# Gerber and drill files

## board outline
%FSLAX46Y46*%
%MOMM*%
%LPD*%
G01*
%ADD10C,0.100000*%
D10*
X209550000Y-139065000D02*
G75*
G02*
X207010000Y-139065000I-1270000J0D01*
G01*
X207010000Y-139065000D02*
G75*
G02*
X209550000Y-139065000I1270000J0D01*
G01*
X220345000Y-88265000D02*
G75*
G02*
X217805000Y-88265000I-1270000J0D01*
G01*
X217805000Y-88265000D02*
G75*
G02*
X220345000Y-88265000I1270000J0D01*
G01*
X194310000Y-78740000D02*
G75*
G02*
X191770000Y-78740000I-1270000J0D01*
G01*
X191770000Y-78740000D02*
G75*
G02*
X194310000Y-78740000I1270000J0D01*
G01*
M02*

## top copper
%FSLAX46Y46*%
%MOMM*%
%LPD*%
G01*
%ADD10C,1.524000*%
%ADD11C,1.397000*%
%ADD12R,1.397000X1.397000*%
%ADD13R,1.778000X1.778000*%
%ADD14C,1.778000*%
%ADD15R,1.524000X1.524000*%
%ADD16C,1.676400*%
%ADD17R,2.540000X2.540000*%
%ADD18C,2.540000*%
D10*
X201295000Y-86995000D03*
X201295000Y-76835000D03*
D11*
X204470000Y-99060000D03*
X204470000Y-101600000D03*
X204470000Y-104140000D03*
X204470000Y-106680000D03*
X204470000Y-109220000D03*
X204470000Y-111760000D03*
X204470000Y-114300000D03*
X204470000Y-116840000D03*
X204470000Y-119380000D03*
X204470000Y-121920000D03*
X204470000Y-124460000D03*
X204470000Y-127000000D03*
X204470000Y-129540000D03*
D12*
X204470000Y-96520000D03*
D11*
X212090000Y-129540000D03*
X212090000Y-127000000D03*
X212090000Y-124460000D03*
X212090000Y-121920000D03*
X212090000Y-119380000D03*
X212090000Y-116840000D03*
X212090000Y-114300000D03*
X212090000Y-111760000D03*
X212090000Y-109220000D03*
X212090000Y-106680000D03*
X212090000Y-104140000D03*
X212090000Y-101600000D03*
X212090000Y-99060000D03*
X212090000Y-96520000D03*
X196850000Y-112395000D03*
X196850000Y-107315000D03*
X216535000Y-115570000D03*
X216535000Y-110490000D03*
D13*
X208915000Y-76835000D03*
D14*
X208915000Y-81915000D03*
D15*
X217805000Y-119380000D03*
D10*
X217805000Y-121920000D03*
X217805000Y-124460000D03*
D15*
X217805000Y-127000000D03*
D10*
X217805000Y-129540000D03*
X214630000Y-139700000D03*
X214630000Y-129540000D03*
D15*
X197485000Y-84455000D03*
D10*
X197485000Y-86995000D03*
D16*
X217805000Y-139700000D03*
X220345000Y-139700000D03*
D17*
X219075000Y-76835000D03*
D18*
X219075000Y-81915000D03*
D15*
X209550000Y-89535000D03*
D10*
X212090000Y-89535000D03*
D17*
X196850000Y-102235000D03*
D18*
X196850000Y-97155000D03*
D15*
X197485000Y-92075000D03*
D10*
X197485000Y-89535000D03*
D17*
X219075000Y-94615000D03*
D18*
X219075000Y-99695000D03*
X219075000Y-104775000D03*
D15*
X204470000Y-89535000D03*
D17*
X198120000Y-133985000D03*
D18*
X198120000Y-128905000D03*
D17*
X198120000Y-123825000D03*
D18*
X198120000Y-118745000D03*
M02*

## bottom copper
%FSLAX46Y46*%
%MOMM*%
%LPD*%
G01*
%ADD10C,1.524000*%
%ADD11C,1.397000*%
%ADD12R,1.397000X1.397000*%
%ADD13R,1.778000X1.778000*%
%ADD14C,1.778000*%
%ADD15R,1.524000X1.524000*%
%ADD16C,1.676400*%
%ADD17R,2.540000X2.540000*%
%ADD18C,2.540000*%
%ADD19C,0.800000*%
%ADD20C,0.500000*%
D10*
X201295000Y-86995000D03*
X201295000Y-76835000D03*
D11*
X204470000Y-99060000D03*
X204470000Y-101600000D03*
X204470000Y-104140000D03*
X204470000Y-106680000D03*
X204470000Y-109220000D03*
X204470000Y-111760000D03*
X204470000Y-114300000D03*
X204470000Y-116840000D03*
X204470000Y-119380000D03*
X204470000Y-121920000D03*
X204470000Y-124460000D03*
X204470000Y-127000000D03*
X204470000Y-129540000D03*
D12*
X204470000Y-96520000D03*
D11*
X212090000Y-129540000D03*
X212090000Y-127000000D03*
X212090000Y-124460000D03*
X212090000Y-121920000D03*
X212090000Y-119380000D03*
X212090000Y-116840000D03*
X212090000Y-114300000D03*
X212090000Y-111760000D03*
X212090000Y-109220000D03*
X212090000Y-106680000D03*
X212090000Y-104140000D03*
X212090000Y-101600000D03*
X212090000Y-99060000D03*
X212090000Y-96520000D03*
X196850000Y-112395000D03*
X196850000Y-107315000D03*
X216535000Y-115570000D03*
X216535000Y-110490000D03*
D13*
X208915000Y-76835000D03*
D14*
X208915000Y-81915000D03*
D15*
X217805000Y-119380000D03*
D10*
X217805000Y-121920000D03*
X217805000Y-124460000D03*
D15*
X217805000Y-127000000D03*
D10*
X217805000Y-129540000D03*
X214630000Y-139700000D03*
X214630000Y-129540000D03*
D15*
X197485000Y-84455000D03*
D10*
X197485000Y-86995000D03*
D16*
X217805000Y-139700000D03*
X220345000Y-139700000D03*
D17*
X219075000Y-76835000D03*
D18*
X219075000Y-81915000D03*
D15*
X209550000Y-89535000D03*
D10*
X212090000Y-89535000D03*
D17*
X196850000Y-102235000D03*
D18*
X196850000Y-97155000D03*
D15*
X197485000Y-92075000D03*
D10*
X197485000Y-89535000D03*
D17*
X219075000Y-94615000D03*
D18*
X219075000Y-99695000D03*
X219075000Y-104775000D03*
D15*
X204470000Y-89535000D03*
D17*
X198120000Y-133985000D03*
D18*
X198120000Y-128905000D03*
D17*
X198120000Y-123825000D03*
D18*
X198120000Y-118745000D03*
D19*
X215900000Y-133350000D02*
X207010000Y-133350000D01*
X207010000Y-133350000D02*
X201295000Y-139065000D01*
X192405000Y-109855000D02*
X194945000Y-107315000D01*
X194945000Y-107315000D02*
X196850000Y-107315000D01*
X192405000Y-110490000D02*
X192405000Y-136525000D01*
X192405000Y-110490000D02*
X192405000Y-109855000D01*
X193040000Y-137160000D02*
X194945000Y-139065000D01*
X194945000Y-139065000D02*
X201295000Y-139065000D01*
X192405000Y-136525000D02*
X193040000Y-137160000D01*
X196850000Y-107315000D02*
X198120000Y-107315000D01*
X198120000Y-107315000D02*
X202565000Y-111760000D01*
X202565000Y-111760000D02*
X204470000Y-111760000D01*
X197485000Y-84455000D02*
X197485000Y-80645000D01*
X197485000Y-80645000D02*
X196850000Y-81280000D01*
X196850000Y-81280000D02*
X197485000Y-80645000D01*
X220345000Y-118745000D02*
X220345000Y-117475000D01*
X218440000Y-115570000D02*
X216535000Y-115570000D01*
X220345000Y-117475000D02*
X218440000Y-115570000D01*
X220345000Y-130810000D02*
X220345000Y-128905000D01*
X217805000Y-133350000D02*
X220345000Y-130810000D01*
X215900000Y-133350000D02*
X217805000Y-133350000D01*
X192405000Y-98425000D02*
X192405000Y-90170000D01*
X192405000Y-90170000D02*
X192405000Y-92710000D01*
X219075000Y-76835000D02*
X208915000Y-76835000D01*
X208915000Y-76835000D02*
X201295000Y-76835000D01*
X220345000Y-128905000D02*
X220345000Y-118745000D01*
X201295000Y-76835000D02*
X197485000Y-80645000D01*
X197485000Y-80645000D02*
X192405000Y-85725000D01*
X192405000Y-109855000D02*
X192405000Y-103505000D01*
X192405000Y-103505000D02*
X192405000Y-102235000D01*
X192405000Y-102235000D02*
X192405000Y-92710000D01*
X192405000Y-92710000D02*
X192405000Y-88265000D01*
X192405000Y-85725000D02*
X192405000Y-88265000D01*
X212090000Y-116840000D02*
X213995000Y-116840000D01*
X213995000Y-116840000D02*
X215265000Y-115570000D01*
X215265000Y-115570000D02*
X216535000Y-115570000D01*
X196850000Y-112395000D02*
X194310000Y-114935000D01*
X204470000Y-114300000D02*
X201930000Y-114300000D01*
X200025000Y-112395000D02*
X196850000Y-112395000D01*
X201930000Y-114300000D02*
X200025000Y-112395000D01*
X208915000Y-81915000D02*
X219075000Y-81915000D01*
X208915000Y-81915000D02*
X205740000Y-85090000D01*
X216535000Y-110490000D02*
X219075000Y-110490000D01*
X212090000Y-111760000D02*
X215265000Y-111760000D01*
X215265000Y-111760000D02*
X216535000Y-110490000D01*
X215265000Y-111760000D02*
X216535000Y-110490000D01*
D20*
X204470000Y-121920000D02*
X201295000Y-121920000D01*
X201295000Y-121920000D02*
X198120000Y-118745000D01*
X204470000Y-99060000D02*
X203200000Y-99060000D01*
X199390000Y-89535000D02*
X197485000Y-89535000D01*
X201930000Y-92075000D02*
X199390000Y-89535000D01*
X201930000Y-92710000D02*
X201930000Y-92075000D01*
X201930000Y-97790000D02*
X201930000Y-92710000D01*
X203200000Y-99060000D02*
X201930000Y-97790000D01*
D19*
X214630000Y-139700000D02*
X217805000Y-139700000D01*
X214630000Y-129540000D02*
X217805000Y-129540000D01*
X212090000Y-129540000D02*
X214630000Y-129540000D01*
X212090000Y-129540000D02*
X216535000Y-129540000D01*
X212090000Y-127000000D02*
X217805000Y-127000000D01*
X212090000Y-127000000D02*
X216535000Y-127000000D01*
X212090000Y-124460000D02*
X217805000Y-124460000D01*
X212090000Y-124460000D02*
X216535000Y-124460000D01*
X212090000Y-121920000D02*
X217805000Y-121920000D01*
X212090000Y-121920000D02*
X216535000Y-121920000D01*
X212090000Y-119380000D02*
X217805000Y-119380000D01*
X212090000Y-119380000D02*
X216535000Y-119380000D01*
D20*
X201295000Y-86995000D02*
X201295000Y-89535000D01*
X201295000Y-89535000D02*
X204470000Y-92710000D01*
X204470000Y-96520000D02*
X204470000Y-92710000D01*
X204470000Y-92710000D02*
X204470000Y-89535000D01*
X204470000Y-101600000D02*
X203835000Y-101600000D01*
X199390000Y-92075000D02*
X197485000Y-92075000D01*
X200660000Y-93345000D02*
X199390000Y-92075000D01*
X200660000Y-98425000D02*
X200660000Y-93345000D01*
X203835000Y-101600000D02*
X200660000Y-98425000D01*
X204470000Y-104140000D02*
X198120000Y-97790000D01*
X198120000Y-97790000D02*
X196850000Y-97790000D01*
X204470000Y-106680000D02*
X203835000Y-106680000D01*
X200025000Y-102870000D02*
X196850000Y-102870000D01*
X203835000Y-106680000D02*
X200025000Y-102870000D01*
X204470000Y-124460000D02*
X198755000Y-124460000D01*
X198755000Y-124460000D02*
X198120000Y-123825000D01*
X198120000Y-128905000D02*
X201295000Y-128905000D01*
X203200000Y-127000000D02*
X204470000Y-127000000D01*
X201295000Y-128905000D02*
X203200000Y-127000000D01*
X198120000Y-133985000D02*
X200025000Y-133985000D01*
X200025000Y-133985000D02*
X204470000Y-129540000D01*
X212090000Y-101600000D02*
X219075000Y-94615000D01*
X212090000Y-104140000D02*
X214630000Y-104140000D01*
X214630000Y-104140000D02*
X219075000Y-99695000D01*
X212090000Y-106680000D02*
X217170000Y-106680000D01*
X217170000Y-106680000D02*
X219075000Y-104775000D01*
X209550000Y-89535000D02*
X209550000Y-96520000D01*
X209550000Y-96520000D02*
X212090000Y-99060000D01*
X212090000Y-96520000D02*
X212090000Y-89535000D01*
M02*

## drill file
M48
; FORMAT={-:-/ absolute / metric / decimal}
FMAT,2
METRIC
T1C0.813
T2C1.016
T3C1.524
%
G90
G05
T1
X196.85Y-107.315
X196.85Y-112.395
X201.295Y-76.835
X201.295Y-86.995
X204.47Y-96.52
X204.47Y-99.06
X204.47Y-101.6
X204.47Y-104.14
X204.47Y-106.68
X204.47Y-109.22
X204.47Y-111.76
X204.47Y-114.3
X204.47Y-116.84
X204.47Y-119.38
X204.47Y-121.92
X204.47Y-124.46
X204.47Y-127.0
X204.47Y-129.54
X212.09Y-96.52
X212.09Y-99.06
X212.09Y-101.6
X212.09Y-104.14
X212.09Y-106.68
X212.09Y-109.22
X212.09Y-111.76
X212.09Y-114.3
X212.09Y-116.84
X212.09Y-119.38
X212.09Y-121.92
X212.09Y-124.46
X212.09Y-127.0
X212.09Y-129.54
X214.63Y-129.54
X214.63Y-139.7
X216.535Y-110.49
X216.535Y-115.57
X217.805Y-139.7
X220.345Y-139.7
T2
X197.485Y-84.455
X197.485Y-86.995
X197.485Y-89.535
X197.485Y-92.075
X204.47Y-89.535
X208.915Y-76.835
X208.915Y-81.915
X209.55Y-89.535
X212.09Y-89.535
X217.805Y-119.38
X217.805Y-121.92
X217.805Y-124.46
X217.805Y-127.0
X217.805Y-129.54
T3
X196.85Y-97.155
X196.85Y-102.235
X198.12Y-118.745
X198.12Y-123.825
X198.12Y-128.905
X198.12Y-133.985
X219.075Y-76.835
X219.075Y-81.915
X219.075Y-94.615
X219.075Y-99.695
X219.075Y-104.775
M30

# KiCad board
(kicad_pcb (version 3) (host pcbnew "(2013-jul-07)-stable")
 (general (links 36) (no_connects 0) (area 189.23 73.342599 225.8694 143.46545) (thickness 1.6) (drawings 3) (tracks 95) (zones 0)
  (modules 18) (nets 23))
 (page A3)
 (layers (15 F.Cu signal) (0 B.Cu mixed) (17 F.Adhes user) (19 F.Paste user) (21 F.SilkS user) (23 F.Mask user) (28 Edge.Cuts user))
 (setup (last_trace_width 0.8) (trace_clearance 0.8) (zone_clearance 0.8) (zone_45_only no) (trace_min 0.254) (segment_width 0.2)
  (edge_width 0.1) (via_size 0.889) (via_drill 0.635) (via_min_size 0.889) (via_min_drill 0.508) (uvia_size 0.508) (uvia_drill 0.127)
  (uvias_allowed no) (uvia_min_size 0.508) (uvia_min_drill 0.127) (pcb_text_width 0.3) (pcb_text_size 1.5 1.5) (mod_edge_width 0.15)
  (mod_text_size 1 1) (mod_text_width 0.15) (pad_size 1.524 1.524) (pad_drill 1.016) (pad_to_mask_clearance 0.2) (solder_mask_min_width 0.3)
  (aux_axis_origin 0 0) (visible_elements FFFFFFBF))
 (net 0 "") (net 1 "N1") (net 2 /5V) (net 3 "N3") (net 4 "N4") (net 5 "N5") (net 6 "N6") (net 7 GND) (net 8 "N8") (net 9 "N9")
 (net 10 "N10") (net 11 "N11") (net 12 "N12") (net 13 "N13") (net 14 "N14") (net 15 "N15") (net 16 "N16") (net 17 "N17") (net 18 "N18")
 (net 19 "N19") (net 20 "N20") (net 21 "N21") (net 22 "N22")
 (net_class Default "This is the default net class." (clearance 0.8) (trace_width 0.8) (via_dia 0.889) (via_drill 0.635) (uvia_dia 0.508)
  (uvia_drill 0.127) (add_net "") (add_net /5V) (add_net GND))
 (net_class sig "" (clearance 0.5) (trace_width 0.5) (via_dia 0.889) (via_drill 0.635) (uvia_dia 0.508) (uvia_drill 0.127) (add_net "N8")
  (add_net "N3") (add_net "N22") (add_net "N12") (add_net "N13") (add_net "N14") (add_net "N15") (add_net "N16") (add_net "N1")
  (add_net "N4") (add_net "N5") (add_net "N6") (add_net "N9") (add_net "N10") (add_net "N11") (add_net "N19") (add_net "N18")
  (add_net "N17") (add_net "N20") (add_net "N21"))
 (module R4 (layer F.Cu) (at 201.295 81.915 90) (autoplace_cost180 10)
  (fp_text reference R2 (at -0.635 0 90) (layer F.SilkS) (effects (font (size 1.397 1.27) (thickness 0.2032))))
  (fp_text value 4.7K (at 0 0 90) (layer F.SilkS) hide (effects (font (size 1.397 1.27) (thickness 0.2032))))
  (pad 1 thru_hole circle (at -5.08 0 90) (size 1.524 1.524) (drill 0.8128) (layers *.Cu *.Mask F.SilkS) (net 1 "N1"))
  (pad 2 thru_hole circle (at 5.08 0 90) (size 1.524 1.524) (drill 0.8128) (layers *.Cu *.Mask F.SilkS) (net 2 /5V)))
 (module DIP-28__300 (layer F.Cu) (at 208.28 113.03 270)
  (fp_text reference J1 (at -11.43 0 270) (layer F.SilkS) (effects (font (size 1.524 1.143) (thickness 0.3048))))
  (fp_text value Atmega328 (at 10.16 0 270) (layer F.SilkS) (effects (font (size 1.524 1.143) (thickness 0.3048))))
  (pad 2 thru_hole circle (at -13.97 3.81 270) (size 1.397 1.397) (drill 0.8128) (layers *.Cu *.Mask F.SilkS) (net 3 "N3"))
  (pad 3 thru_hole circle (at -11.43 3.81 270) (size 1.397 1.397) (drill 0.8128) (layers *.Cu *.Mask F.SilkS) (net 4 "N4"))
  (pad 4 thru_hole circle (at -8.89 3.81 270) (size 1.397 1.397) (drill 0.8128) (layers *.Cu *.Mask F.SilkS) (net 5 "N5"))
  (pad 5 thru_hole circle (at -6.35 3.81 270) (size 1.397 1.397) (drill 0.8128) (layers *.Cu *.Mask F.SilkS) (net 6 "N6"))
  (pad 6 thru_hole circle (at -3.81 3.81 270) (size 1.397 1.397) (drill 0.8128) (layers *.Cu *.Mask F.SilkS))
  (pad 7 thru_hole circle (at -1.27 3.81 270) (size 1.397 1.397) (drill 0.8128) (layers *.Cu *.Mask F.SilkS) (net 2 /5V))
  (pad 8 thru_hole circle (at 1.27 3.81 270) (size 1.397 1.397) (drill 0.8128) (layers *.Cu *.Mask F.SilkS) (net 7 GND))
  (pad 9 thru_hole circle (at 3.81 3.81 270) (size 1.397 1.397) (drill 0.8128) (layers *.Cu *.Mask F.SilkS))
  (pad 10 thru_hole circle (at 6.35 3.81 270) (size 1.397 1.397) (drill 0.8128) (layers *.Cu *.Mask F.SilkS))
  (pad 11 thru_hole circle (at 8.89 3.81 270) (size 1.397 1.397) (drill 0.8128) (layers *.Cu *.Mask F.SilkS) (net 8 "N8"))
  (pad 12 thru_hole circle (at 11.43 3.81 270) (size 1.397 1.397) (drill 0.8128) (layers *.Cu *.Mask F.SilkS) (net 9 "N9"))
  (pad 13 thru_hole circle (at 13.97 3.81 270) (size 1.397 1.397) (drill 0.8128) (layers *.Cu *.Mask F.SilkS) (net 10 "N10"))
  (pad 14 thru_hole circle (at 16.51 3.81 270) (size 1.397 1.397) (drill 0.8128) (layers *.Cu *.Mask F.SilkS) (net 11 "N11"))
  (pad 1 thru_hole rect (at -16.51 3.81 270) (size 1.397 1.397) (drill 0.8128) (layers *.Cu *.Mask F.SilkS) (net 1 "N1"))
  (pad 15 thru_hole circle (at 16.51 -3.81 270) (size 1.397 1.397) (drill 0.8128) (layers *.Cu *.Mask F.SilkS) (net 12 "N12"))
  (pad 16 thru_hole circle (at 13.97 -3.81 270) (size 1.397 1.397) (drill 0.8128) (layers *.Cu *.Mask F.SilkS) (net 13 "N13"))
  (pad 17 thru_hole circle (at 11.43 -3.81 270) (size 1.397 1.397) (drill 0.8128) (layers *.Cu *.Mask F.SilkS) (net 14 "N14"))
  (pad 18 thru_hole circle (at 8.89 -3.81 270) (size 1.397 1.397) (drill 0.8128) (layers *.Cu *.Mask F.SilkS) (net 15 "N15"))
  (pad 19 thru_hole circle (at 6.35 -3.81 270) (size 1.397 1.397) (drill 0.8128) (layers *.Cu *.Mask F.SilkS) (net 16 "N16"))
  (pad 20 thru_hole circle (at 3.81 -3.81 270) (size 1.397 1.397) (drill 0.8128) (layers *.Cu *.Mask F.SilkS) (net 2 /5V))
  (pad 21 thru_hole circle (at 1.27 -3.81 270) (size 1.397 1.397) (drill 0.8128) (layers *.Cu *.Mask F.SilkS))
  (pad 22 thru_hole circle (at -1.27 -3.81 270) (size 1.397 1.397) (drill 0.8128) (layers *.Cu *.Mask F.SilkS) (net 7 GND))
  (pad 23 thru_hole circle (at -3.81 -3.81 270) (size 1.397 1.397) (drill 0.8128) (layers *.Cu *.Mask F.SilkS))
  (pad 24 thru_hole circle (at -6.35 -3.81 270) (size 1.397 1.397) (drill 0.8128) (layers *.Cu *.Mask F.SilkS) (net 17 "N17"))
  (pad 25 thru_hole circle (at -8.89 -3.81 270) (size 1.397 1.397) (drill 0.8128) (layers *.Cu *.Mask F.SilkS) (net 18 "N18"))
  (pad 26 thru_hole circle (at -11.43 -3.81 270) (size 1.397 1.397) (drill 0.8128) (layers *.Cu *.Mask F.SilkS) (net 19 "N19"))
  (pad 27 thru_hole circle (at -13.97 -3.81 270) (size 1.397 1.397) (drill 0.8128) (layers *.Cu *.Mask F.SilkS) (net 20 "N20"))
  (pad 28 thru_hole circle (at -16.51 -3.81 270) (size 1.397 1.397) (drill 0.8128) (layers *.Cu *.Mask F.SilkS) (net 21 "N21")))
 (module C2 (layer F.Cu) (at 196.85 109.855 90)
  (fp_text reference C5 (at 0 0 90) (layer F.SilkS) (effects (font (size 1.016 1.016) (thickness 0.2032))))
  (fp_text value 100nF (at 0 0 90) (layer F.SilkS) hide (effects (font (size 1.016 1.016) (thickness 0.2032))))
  (pad 1 thru_hole circle (at -2.54 0 90) (size 1.397 1.397) (drill 0.8128) (layers *.Cu *.Mask F.SilkS) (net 7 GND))
  (pad 2 thru_hole circle (at 2.54 0 90) (size 1.397 1.397) (drill 0.8128) (layers *.Cu *.Mask F.SilkS) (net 2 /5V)))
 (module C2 (layer F.Cu) (at 216.535 113.03 90)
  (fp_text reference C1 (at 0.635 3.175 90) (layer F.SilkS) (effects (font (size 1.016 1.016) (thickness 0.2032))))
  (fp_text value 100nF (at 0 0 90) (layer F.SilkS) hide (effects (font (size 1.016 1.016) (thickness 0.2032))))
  (pad 1 thru_hole circle (at -2.54 0 90) (size 1.397 1.397) (drill 0.8128) (layers *.Cu *.Mask F.SilkS) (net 2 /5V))
  (pad 2 thru_hole circle (at 2.54 0 90) (size 1.397 1.397) (drill 0.8128) (layers *.Cu *.Mask F.SilkS) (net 7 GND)))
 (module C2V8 (layer F.Cu) (at 208.915 79.375 270)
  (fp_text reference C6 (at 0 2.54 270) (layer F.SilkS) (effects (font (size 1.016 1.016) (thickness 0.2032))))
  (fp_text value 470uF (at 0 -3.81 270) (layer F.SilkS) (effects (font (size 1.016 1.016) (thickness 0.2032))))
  (pad 1 thru_hole rect (at -2.54 0 270) (size 1.778 1.778) (drill 1.016) (layers *.Cu *.Mask F.SilkS) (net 2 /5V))
  (pad 2 thru_hole circle (at 2.54 0 270) (size 1.778 1.778) (drill 1.016) (layers *.Cu *.Mask F.SilkS) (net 7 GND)))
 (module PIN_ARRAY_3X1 (layer F.Cu) (at 217.805 121.92 270)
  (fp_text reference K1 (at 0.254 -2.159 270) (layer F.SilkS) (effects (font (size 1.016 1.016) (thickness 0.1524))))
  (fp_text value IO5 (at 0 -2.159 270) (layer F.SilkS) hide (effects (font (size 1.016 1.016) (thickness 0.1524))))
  (pad 1 thru_hole rect (at -2.54 0 270) (size 1.524 1.524) (drill 1.016) (layers *.Cu *.Mask F.SilkS) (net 16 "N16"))
  (pad 2 thru_hole circle (at 0 0 270) (size 1.524 1.524) (drill 1.016) (layers *.Cu *.Mask F.SilkS) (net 15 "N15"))
  (pad 3 thru_hole circle (at 2.54 0 270) (size 1.524 1.524) (drill 1.016) (layers *.Cu *.Mask F.SilkS) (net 14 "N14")))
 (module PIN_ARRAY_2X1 (layer F.Cu) (at 217.805 128.27 270)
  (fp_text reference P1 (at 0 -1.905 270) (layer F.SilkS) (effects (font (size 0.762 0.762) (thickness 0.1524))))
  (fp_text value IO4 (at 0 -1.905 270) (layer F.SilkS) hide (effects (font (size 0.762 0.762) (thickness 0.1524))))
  (pad 1 thru_hole rect (at -1.27 0 270) (size 1.524 1.524) (drill 1.016) (layers *.Cu *.Mask F.SilkS) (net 13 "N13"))
  (pad 2 thru_hole circle (at 1.27 0 270) (size 1.524 1.524) (drill 1.016) (layers *.Cu *.Mask F.SilkS) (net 12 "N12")))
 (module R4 (layer F.Cu) (at 214.63 134.62 90) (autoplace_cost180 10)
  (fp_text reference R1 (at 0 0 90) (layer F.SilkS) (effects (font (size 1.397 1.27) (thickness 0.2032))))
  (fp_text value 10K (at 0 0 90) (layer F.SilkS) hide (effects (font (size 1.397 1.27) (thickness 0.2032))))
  (pad 1 thru_hole circle (at -5.08 0 90) (size 1.524 1.524) (drill 0.8128) (layers *.Cu *.Mask F.SilkS) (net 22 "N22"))
  (pad 2 thru_hole circle (at 5.08 0 90) (size 1.524 1.524) (drill 0.8128) (layers *.Cu *.Mask F.SilkS) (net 12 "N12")))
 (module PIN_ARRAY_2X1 (layer F.Cu) (at 197.485 85.725 270)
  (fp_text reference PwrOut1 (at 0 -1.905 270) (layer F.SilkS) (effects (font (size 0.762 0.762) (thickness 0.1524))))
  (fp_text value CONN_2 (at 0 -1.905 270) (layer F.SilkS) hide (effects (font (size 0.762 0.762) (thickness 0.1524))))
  (pad 1 thru_hole rect (at -1.27 0 270) (size 1.524 1.524) (drill 1.016) (layers *.Cu *.Mask F.SilkS) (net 2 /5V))
  (pad 2 thru_hole circle (at 1.27 0 270) (size 1.524 1.524) (drill 1.016) (layers *.Cu *.Mask F.SilkS) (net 7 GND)))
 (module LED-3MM (layer F.Cu) (at 219.075 139.7)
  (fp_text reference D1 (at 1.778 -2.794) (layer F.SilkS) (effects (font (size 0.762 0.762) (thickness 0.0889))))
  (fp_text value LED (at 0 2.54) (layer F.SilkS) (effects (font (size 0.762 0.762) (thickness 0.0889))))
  (pad 1 thru_hole circle (at -1.27 0) (size 1.6764 1.6764) (drill 0.8128) (layers *.Cu *.Mask F.SilkS) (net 22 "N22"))
  (pad 2 thru_hole circle (at 1.27 0) (size 1.6764 1.6764) (drill 0.8128) (layers *.Cu *.Mask F.SilkS) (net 7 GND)))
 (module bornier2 (layer F.Cu) (at 219.075 79.375 270)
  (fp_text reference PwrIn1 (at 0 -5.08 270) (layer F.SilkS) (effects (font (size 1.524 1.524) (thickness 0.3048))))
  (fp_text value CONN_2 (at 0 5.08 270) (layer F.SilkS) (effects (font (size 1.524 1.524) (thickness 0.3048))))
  (pad 1 thru_hole rect (at -2.54 0 270) (size 2.54 2.54) (drill 1.524) (layers *.Cu *.Mask F.SilkS) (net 2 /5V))
  (pad 2 thru_hole circle (at 2.54 0 270) (size 2.54 2.54) (drill 1.524) (layers *.Cu *.Mask F.SilkS) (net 7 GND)))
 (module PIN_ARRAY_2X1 (layer F.Cu) (at 210.82 89.535)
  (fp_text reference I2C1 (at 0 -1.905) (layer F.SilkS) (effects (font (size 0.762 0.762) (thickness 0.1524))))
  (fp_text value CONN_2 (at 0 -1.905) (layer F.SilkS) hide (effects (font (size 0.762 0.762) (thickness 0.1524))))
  (pad 1 thru_hole rect (at -1.27 0) (size 1.524 1.524) (drill 1.016) (layers *.Cu *.Mask F.SilkS) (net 20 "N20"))
  (pad 2 thru_hole circle (at 1.27 0) (size 1.524 1.524) (drill 1.016) (layers *.Cu *.Mask F.SilkS) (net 21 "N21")))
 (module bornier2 (layer F.Cu) (at 196.85 99.695 90)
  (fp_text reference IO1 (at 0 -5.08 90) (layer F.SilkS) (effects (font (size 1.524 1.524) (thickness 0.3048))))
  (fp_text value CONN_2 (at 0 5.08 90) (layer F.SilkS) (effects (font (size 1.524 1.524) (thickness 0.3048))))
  (pad 1 thru_hole rect (at -2.54 0 90) (size 2.54 2.54) (drill 1.524) (layers *.Cu *.Mask F.SilkS) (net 6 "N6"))
  (pad 2 thru_hole circle (at 2.54 0 90) (size 2.54 2.54) (drill 1.524) (layers *.Cu *.Mask F.SilkS) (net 5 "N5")))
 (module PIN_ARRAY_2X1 (layer F.Cu) (at 197.485 90.805 90)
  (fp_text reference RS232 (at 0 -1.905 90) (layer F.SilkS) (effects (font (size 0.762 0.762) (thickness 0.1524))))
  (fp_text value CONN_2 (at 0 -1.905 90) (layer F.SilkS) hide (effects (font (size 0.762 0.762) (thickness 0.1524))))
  (pad 1 thru_hole rect (at -1.27 0 90) (size 1.524 1.524) (drill 1.016) (layers *.Cu *.Mask F.SilkS) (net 4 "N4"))
  (pad 2 thru_hole circle (at 1.27 0 90) (size 1.524 1.524) (drill 1.016) (layers *.Cu *.Mask F.SilkS) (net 3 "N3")))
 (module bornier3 (layer F.Cu) (at 219.075 99.695 270)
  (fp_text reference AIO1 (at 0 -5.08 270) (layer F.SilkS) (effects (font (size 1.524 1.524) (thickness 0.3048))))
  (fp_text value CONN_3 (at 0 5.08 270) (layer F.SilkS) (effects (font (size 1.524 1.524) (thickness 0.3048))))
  (pad 1 thru_hole rect (at -5.08 0 270) (size 2.54 2.54) (drill 1.524) (layers *.Cu *.Mask F.SilkS) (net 19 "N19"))
  (pad 2 thru_hole circle (at 0 0 270) (size 2.54 2.54) (drill 1.524) (layers *.Cu *.Mask F.SilkS) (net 18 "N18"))
  (pad 3 thru_hole circle (at 5.08 0 270) (size 2.54 2.54) (drill 1.524) (layers *.Cu *.Mask F.SilkS) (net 17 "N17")))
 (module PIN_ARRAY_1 (layer F.Cu) (at 204.47 89.535)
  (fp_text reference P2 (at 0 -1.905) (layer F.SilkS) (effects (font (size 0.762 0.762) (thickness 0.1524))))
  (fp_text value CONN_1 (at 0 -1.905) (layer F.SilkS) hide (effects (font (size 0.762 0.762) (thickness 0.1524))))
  (pad 1 thru_hole rect (at 0 0) (size 1.524 1.524) (drill 1.016) (layers *.Cu *.Mask F.SilkS) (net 1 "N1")))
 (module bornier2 (layer F.Cu) (at 198.12 131.445 90)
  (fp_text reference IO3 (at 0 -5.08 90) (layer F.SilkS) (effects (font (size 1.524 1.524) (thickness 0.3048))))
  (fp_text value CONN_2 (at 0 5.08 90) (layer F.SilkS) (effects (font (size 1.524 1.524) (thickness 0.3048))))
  (pad 1 thru_hole rect (at -2.54 0 90) (size 2.54 2.54) (drill 1.524) (layers *.Cu *.Mask F.SilkS) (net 11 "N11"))
  (pad 2 thru_hole circle (at 2.54 0 90) (size 2.54 2.54) (drill 1.524) (layers *.Cu *.Mask F.SilkS) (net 10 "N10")))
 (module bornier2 (layer F.Cu) (at 198.12 121.285 90)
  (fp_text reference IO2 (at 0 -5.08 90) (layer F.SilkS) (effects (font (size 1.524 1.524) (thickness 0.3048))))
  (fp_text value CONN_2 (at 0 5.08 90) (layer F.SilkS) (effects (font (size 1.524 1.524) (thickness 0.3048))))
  (pad 1 thru_hole rect (at -2.54 0 90) (size 2.54 2.54) (drill 1.524) (layers *.Cu *.Mask F.SilkS) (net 9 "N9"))
  (pad 2 thru_hole circle (at 2.54 0 90) (size 2.54 2.54) (drill 1.524) (layers *.Cu *.Mask F.SilkS) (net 8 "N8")))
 (gr_circle (center 208.28 139.065) (end 209.55 139.065) (layer Edge.Cuts) (width 0.1))
 (gr_circle (center 219.075 88.265) (end 217.805 88.265) (layer Edge.Cuts) (width 0.1))
 (gr_circle (center 193.04 78.74) (end 194.31 78.74) (layer Edge.Cuts) (width 0.1))
 (segment (start 215.9 133.35) (end 207.01 133.35) (width 0.8) (layer B.Cu) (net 2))
 (segment (start 207.01 133.35) (end 201.295 139.065) (width 0.8) (layer B.Cu) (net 2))
 (segment (start 192.405 109.855) (end 194.945 107.315) (width 0.8) (layer B.Cu) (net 2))
 (segment (start 194.945 107.315) (end 196.85 107.315) (width 0.8) (layer B.Cu) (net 2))
 (segment (start 192.405 110.49) (end 192.405 136.525) (width 0.8) (layer B.Cu) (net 2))
 (segment (start 192.405 110.49) (end 192.405 109.855) (width 0.8) (layer B.Cu) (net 2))
 (segment (start 193.04 137.16) (end 194.945 139.065) (width 0.8) (layer B.Cu) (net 2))
 (segment (start 194.945 139.065) (end 201.295 139.065) (width 0.8) (layer B.Cu) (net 2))
 (segment (start 192.405 136.525) (end 193.04 137.16) (width 0.8) (layer B.Cu) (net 2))
 (segment (start 196.85 107.315) (end 198.12 107.315) (width 0.8) (layer B.Cu) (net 2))
 (segment (start 198.12 107.315) (end 202.565 111.76) (width 0.8) (layer B.Cu) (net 2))
 (segment (start 202.565 111.76) (end 204.47 111.76) (width 0.8) (layer B.Cu) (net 2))
 (segment (start 197.485 84.455) (end 197.485 80.645) (width 0.8) (layer B.Cu) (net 2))
 (segment (start 197.485 80.645) (end 196.85 81.28) (width 0.8) (layer B.Cu) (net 2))
 (segment (start 196.85 81.28) (end 197.485 80.645) (width 0.8) (layer B.Cu) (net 2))
 (segment (start 220.345 118.745) (end 220.345 117.475) (width 0.8) (layer B.Cu) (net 2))
 (segment (start 218.44 115.57) (end 216.535 115.57) (width 0.8) (layer B.Cu) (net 2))
 (segment (start 220.345 117.475) (end 218.44 115.57) (width 0.8) (layer B.Cu) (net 2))
 (segment (start 220.345 130.81) (end 220.345 128.905) (width 0.8) (layer B.Cu) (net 2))
 (segment (start 217.805 133.35) (end 220.345 130.81) (width 0.8) (layer B.Cu) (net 2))
 (segment (start 215.9 133.35) (end 217.805 133.35) (width 0.8) (layer B.Cu) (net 2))
 (segment (start 192.405 98.425) (end 192.405 90.17) (width 0.8) (layer B.Cu) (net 2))
 (segment (start 192.405 90.17) (end 192.405 92.71) (width 0.8) (layer B.Cu) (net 2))
 (segment (start 219.075 76.835) (end 208.915 76.835) (width 0.8) (layer B.Cu) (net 2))
 (segment (start 208.915 76.835) (end 201.295 76.835) (width 0.8) (layer B.Cu) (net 2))
 (segment (start 220.345 128.905) (end 220.345 118.745) (width 0.8) (layer B.Cu) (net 2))
 (segment (start 201.295 76.835) (end 197.485 80.645) (width 0.8) (layer B.Cu) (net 2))
 (segment (start 197.485 80.645) (end 192.405 85.725) (width 0.8) (layer B.Cu) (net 2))
 (segment (start 192.405 109.855) (end 192.405 103.505) (width 0.8) (layer B.Cu) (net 2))
 (segment (start 192.405 103.505) (end 192.405 102.235) (width 0.8) (layer B.Cu) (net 2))
 (segment (start 192.405 102.235) (end 192.405 92.71) (width 0.8) (layer B.Cu) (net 2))
 (segment (start 192.405 92.71) (end 192.405 88.265) (width 0.8) (layer B.Cu) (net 2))
 (segment (start 192.405 85.725) (end 192.405 88.265) (width 0.8) (layer B.Cu) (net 2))
 (segment (start 212.09 116.84) (end 213.995 116.84) (width 0.8) (layer B.Cu) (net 2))
 (segment (start 213.995 116.84) (end 215.265 115.57) (width 0.8) (layer B.Cu) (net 2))
 (segment (start 215.265 115.57) (end 216.535 115.57) (width 0.8) (layer B.Cu) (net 2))
 (segment (start 196.85 112.395) (end 194.31 114.935) (width 0.8) (layer B.Cu) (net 7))
 (segment (start 204.47 114.3) (end 201.93 114.3) (width 0.8) (layer B.Cu) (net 7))
 (segment (start 200.025 112.395) (end 196.85 112.395) (width 0.8) (layer B.Cu) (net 7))
 (segment (start 201.93 114.3) (end 200.025 112.395) (width 0.8) (layer B.Cu) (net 7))
 (segment (start 208.915 81.915) (end 219.075 81.915) (width 0.8) (layer B.Cu) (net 7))
 (segment (start 208.915 81.915) (end 205.74 85.09) (width 0.8) (layer B.Cu) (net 7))
 (segment (start 216.535 110.49) (end 219.075 110.49) (width 0.8) (layer B.Cu) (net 7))
 (segment (start 212.09 111.76) (end 215.265 111.76) (width 0.8) (layer B.Cu) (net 7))
 (segment (start 215.265 111.76) (end 216.535 110.49) (width 0.8) (layer B.Cu) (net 7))
 (segment (start 215.265 111.76) (end 216.535 110.49) (width 0.8) (layer B.Cu) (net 7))
 (segment (start 204.47 121.92) (end 201.295 121.92) (width 0.5) (layer B.Cu) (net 8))
 (segment (start 201.295 121.92) (end 198.12 118.745) (width 0.5) (layer B.Cu) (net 8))
 (segment (start 204.47 99.06) (end 203.2 99.06) (width 0.5) (layer B.Cu) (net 3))
 (segment (start 199.39 89.535) (end 197.485 89.535) (width 0.5) (layer B.Cu) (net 3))
 (segment (start 201.93 92.075) (end 199.39 89.535) (width 0.5) (layer B.Cu) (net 3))
 (segment (start 201.93 92.71) (end 201.93 92.075) (width 0.5) (layer B.Cu) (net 3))
 (segment (start 201.93 97.79) (end 201.93 92.71) (width 0.5) (layer B.Cu) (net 3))
 (segment (start 203.2 99.06) (end 201.93 97.79) (width 0.5) (layer B.Cu) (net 3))
 (segment (start 214.63 139.7) (end 217.805 139.7) (width 0.8) (layer B.Cu) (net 22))
 (segment (start 214.63 129.54) (end 217.805 129.54) (width 0.8) (layer B.Cu) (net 12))
 (segment (start 212.09 129.54) (end 214.63 129.54) (width 0.8) (layer B.Cu) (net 12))
 (segment (start 212.09 129.54) (end 216.535 129.54) (width 0.8) (layer B.Cu) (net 12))
 (segment (start 212.09 127) (end 217.805 127) (width 0.8) (layer B.Cu) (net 13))
 (segment (start 212.09 127) (end 216.535 127) (width 0.8) (layer B.Cu) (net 13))
 (segment (start 212.09 124.46) (end 217.805 124.46) (width 0.8) (layer B.Cu) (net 14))
 (segment (start 212.09 124.46) (end 216.535 124.46) (width 0.8) (layer B.Cu) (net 14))
 (segment (start 212.09 121.92) (end 217.805 121.92) (width 0.8) (layer B.Cu) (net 15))
 (segment (start 212.09 121.92) (end 216.535 121.92) (width 0.8) (layer B.Cu) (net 15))
 (segment (start 212.09 119.38) (end 217.805 119.38) (width 0.8) (layer B.Cu) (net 16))
 (segment (start 212.09 119.38) (end 216.535 119.38) (width 0.8) (layer B.Cu) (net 16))
 (segment (start 201.295 86.995) (end 201.295 89.535) (width 0.5) (layer B.Cu) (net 1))
 (segment (start 201.295 89.535) (end 204.47 92.71) (width 0.5) (layer B.Cu) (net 1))
 (segment (start 204.47 96.52) (end 204.47 92.71) (width 0.5) (layer B.Cu) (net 1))
 (segment (start 204.47 92.71) (end 204.47 89.535) (width 0.5) (layer B.Cu) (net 1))
 (segment (start 204.47 101.6) (end 203.835 101.6) (width 0.5) (layer B.Cu) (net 4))
 (segment (start 199.39 92.075) (end 197.485 92.075) (width 0.5) (layer B.Cu) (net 4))
 (segment (start 200.66 93.345) (end 199.39 92.075) (width 0.5) (layer B.Cu) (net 4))
 (segment (start 200.66 98.425) (end 200.66 93.345) (width 0.5) (layer B.Cu) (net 4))
 (segment (start 203.835 101.6) (end 200.66 98.425) (width 0.5) (layer B.Cu) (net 4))
 (segment (start 204.47 104.14) (end 198.12 97.79) (width 0.5) (layer B.Cu) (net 5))
 (segment (start 198.12 97.79) (end 196.85 97.79) (width 0.5) (layer B.Cu) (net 5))
 (segment (start 204.47 106.68) (end 203.835 106.68) (width 0.5) (layer B.Cu) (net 6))
 (segment (start 200.025 102.87) (end 196.85 102.87) (width 0.5) (layer B.Cu) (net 6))
 (segment (start 203.835 106.68) (end 200.025 102.87) (width 0.5) (layer B.Cu) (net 6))
 (segment (start 204.47 124.46) (end 198.755 124.46) (width 0.5) (layer B.Cu) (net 9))
 (segment (start 198.755 124.46) (end 198.12 123.825) (width 0.5) (layer B.Cu) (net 9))
 (segment (start 198.12 128.905) (end 201.295 128.905) (width 0.5) (layer B.Cu) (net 10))
 (segment (start 203.2 127) (end 204.47 127) (width 0.5) (layer B.Cu) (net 10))
 (segment (start 201.295 128.905) (end 203.2 127) (width 0.5) (layer B.Cu) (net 10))
 (segment (start 198.12 133.985) (end 200.025 133.985) (width 0.5) (layer B.Cu) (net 11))
 (segment (start 200.025 133.985) (end 204.47 129.54) (width 0.5) (layer B.Cu) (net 11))
 (segment (start 212.09 101.6) (end 219.075 94.615) (width 0.5) (layer B.Cu) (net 19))
 (segment (start 212.09 104.14) (end 214.63 104.14) (width 0.5) (layer B.Cu) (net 18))
 (segment (start 214.63 104.14) (end 219.075 99.695) (width 0.5) (layer B.Cu) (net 18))
 (segment (start 212.09 106.68) (end 217.17 106.68) (width 0.5) (layer B.Cu) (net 17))
 (segment (start 217.17 106.68) (end 219.075 104.775) (width 0.5) (layer B.Cu) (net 17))
 (segment (start 209.55 89.535) (end 209.55 96.52) (width 0.5) (layer B.Cu) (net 20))
 (segment (start 209.55 96.52) (end 212.09 99.06) (width 0.5) (layer B.Cu) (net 20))
 (segment (start 212.09 96.52) (end 212.09 89.535) (width 0.5) (layer B.Cu) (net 21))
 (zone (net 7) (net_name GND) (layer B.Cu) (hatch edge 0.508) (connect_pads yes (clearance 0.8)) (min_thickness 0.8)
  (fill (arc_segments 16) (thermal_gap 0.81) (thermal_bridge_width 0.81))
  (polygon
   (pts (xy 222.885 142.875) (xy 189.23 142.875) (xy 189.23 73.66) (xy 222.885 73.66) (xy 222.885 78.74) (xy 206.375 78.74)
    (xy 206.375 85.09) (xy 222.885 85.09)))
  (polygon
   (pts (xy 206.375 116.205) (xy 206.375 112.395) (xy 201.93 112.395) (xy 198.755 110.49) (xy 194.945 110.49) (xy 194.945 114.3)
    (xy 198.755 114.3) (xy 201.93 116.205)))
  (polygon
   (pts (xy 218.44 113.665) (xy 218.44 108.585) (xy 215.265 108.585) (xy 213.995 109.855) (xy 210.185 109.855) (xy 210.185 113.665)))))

